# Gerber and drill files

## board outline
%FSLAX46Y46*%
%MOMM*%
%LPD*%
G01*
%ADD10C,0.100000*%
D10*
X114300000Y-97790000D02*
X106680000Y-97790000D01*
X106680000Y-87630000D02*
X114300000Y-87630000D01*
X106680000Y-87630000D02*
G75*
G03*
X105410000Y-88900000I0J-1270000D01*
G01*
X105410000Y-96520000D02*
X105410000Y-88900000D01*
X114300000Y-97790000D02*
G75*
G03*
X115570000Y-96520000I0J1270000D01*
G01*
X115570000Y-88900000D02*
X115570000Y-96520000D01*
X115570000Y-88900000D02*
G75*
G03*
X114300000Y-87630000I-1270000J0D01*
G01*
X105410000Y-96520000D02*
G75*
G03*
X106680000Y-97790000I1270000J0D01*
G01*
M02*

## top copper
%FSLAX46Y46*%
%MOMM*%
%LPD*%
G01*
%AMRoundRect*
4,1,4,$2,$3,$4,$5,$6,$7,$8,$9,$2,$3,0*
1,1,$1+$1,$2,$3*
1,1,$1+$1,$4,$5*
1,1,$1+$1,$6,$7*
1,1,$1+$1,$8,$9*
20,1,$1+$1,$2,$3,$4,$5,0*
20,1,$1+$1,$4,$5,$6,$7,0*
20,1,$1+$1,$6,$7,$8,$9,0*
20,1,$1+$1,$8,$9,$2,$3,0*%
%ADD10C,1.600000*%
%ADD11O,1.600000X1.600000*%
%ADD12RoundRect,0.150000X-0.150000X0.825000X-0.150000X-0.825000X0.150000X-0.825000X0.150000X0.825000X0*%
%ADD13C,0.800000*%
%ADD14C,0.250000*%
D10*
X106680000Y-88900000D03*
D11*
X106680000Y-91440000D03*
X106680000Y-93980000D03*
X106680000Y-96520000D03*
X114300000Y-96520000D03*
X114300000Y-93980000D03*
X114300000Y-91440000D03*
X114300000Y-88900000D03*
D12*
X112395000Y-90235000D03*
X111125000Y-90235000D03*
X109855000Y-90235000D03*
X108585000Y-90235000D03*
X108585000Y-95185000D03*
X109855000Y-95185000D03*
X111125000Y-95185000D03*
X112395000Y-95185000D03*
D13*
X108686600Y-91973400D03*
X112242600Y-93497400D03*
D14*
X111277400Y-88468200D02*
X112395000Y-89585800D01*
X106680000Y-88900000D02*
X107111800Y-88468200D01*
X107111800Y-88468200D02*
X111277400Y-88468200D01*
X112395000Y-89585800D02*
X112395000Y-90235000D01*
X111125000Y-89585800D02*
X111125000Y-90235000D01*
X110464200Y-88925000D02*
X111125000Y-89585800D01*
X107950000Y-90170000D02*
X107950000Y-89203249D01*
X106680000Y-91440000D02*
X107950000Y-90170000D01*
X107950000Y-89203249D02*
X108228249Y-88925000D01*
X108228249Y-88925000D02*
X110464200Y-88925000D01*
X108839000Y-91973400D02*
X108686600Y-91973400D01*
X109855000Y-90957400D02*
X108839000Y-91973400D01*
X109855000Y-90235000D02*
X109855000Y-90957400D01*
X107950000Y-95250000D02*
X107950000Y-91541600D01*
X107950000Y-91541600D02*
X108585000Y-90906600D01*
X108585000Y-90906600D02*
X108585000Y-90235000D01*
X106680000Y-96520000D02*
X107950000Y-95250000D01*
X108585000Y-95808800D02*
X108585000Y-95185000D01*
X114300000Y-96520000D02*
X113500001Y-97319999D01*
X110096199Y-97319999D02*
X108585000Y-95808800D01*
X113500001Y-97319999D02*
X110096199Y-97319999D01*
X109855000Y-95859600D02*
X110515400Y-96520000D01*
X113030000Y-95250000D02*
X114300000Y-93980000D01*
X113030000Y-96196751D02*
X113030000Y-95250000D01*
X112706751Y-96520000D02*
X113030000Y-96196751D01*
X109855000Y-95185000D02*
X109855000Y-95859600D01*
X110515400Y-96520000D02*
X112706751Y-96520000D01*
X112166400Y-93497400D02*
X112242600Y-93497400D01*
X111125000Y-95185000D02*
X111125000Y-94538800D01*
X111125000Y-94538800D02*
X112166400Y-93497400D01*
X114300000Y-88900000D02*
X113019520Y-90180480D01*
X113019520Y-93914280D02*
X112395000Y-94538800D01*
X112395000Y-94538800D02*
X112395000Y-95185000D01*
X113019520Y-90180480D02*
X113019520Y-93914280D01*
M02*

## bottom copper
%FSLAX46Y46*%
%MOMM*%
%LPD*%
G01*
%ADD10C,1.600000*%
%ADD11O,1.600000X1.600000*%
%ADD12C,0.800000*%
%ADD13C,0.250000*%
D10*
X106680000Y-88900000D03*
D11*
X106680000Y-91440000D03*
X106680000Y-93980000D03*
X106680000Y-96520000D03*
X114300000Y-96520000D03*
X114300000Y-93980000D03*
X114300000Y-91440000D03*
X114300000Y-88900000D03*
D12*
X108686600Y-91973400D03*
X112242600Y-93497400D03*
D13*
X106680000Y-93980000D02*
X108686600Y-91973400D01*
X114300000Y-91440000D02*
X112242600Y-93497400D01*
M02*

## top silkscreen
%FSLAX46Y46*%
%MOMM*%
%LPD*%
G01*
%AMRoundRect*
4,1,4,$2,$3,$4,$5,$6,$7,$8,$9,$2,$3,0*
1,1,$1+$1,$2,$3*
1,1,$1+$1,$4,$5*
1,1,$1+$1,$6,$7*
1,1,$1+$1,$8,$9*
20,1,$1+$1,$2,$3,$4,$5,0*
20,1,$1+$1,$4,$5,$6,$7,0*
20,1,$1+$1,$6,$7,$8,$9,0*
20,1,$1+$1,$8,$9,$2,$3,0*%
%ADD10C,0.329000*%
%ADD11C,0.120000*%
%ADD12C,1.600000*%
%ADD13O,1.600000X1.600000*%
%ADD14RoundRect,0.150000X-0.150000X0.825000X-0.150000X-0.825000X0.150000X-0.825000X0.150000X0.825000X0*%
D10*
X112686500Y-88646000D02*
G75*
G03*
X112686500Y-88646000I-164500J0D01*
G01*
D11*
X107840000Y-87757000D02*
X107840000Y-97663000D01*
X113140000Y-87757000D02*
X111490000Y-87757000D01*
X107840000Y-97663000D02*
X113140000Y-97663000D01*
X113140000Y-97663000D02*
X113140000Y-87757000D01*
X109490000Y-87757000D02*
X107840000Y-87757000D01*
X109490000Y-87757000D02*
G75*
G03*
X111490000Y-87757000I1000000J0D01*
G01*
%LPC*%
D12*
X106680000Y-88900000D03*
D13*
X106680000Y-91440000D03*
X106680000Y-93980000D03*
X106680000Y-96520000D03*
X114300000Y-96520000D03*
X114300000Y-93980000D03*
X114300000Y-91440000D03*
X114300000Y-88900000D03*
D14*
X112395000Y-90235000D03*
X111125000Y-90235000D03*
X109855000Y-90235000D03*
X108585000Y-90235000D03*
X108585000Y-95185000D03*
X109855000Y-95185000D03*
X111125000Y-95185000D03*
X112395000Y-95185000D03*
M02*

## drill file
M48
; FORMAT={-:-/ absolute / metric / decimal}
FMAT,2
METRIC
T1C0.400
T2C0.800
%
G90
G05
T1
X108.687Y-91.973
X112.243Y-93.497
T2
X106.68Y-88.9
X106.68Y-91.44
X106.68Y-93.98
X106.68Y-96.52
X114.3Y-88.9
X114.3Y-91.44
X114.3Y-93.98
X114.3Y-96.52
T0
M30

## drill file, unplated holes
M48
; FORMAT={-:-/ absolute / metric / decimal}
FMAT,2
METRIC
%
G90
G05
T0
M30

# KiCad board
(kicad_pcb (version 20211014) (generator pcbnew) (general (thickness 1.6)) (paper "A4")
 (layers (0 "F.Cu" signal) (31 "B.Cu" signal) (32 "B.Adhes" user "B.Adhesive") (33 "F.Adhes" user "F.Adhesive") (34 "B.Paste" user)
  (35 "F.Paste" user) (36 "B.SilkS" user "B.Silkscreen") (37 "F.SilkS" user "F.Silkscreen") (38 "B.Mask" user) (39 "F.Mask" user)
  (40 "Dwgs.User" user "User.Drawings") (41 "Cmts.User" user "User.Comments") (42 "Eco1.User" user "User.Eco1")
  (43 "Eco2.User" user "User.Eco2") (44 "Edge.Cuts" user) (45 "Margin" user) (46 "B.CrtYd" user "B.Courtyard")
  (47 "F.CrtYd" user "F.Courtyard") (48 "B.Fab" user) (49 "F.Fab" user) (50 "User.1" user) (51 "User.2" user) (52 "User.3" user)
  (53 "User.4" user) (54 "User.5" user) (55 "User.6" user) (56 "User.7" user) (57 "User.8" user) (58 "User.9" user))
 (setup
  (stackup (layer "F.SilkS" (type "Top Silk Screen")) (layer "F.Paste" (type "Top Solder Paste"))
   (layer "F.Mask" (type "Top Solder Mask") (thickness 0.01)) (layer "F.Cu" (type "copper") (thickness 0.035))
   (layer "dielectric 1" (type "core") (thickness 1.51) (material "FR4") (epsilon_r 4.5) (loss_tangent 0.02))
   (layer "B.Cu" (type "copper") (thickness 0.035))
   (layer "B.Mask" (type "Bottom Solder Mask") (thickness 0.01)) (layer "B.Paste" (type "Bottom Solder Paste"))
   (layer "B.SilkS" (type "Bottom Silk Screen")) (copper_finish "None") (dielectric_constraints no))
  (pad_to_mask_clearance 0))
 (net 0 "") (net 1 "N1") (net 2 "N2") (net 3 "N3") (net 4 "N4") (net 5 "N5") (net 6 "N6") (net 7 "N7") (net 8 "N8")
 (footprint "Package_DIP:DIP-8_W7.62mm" (layer "F.Cu") (at 106.68 88.9)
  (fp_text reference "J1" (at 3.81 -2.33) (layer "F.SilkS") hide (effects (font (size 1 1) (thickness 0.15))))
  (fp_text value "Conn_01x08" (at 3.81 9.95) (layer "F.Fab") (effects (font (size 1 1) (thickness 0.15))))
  (fp_line (start 1.16 -1.143) (end 1.16 8.763) (layer "F.SilkS") (width 0.12))
  (fp_line (start 6.46 -1.143) (end 4.81 -1.143) (layer "F.SilkS") (width 0.12))
  (fp_line (start 1.16 8.763) (end 6.46 8.763) (layer "F.SilkS") (width 0.12))
  (fp_line (start 6.46 8.763) (end 6.46 -1.143) (layer "F.SilkS") (width 0.12))
  (fp_line (start 2.81 -1.143) (end 1.16 -1.143) (layer "F.SilkS") (width 0.12))
  (fp_arc (start 4.81 -1.143) (mid 3.81 -0.143) (end 2.81 -1.143) (layer "F.SilkS") (width 0.12))
  (pad "1" thru_hole circle (at 0 0) (size 1.6 1.6) (drill 0.8) (layers *.Cu *.Mask) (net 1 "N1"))
  (pad "2" thru_hole oval (at 0 2.54) (size 1.6 1.6) (drill 0.8) (layers *.Cu *.Mask) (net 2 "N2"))
  (pad "3" thru_hole oval (at 0 5.08) (size 1.6 1.6) (drill 0.8) (layers *.Cu *.Mask) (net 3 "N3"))
  (pad "4" thru_hole oval (at 0 7.62) (size 1.6 1.6) (drill 0.8) (layers *.Cu *.Mask) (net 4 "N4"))
  (pad "5" thru_hole oval (at 7.62 7.62) (size 1.6 1.6) (drill 0.8) (layers *.Cu *.Mask) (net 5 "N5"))
  (pad "6" thru_hole oval (at 7.62 5.08) (size 1.6 1.6) (drill 0.8) (layers *.Cu *.Mask) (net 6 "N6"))
  (pad "7" thru_hole oval (at 7.62 2.54) (size 1.6 1.6) (drill 0.8) (layers *.Cu *.Mask) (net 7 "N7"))
  (pad "8" thru_hole oval (at 7.62 0) (size 1.6 1.6) (drill 0.8) (layers *.Cu *.Mask) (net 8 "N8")))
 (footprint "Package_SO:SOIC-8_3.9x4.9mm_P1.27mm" (layer "F.Cu") (at 110.49 92.71 -90)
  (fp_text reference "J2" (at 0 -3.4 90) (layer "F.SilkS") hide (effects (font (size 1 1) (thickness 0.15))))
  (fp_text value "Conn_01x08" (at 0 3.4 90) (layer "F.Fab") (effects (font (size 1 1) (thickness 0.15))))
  (pad "1" smd roundrect (at -2.475 -1.905 270) (size 1.95 0.6) (layers "F.Cu" "F.Paste" "F.Mask") (roundrect_rratio 0.25) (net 1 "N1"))
  (pad "2" smd roundrect (at -2.475 -0.635 270) (size 1.95 0.6) (layers "F.Cu" "F.Paste" "F.Mask") (roundrect_rratio 0.25) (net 2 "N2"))
  (pad "3" smd roundrect (at -2.475 0.635 270) (size 1.95 0.6) (layers "F.Cu" "F.Paste" "F.Mask") (roundrect_rratio 0.25) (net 3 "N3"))
  (pad "4" smd roundrect (at -2.475 1.905 270) (size 1.95 0.6) (layers "F.Cu" "F.Paste" "F.Mask") (roundrect_rratio 0.25) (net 4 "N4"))
  (pad "5" smd roundrect (at 2.475 1.905 270) (size 1.95 0.6) (layers "F.Cu" "F.Paste" "F.Mask") (roundrect_rratio 0.25) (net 5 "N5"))
  (pad "6" smd roundrect (at 2.475 0.635 270) (size 1.95 0.6) (layers "F.Cu" "F.Paste" "F.Mask") (roundrect_rratio 0.25) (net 6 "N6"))
  (pad "7" smd roundrect (at 2.475 -0.635 270) (size 1.95 0.6) (layers "F.Cu" "F.Paste" "F.Mask") (roundrect_rratio 0.25) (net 7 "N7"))
  (pad "8" smd roundrect (at 2.475 -1.905 270) (size 1.95 0.6) (layers "F.Cu" "F.Paste" "F.Mask") (roundrect_rratio 0.25) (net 8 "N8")))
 (gr_circle (center 112.522 88.646) (end 112.776 88.646) (layer "F.SilkS") (width 0.15) (fill solid))
 (gr_line (start 114.3 97.79) (end 106.68 97.79) (layer "Edge.Cuts") (width 0.1))
 (gr_line (start 106.68 87.63) (end 114.3 87.63) (layer "Edge.Cuts") (width 0.1))
 (gr_arc (start 105.41 88.9) (mid 105.781974 88.001974) (end 106.68 87.63) (layer "Edge.Cuts") (width 0.1))
 (gr_line (start 105.41 96.52) (end 105.41 88.9) (layer "Edge.Cuts") (width 0.1))
 (gr_arc (start 115.57 96.52) (mid 115.198026 97.418026) (end 114.3 97.79) (layer "Edge.Cuts") (width 0.1))
 (gr_line (start 115.57 88.9) (end 115.57 96.52) (layer "Edge.Cuts") (width 0.1))
 (gr_arc (start 114.3 87.63) (mid 115.198026 88.001974) (end 115.57 88.9) (layer "Edge.Cuts") (width 0.1))
 (gr_arc (start 106.68 97.79) (mid 105.781974 97.418026) (end 105.41 96.52) (layer "Edge.Cuts") (width 0.1))
 (segment (start 111.2774 88.4682) (end 112.395 89.5858) (width 0.25) (layer "F.Cu") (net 1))
 (segment (start 106.68 88.9) (end 107.1118 88.4682) (width 0.25) (layer "F.Cu") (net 1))
 (segment (start 107.1118 88.4682) (end 111.2774 88.4682) (width 0.25) (layer "F.Cu") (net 1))
 (segment (start 112.395 89.5858) (end 112.395 90.235) (width 0.25) (layer "F.Cu") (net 1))
 (segment (start 111.125 89.5858) (end 111.125 90.235) (width 0.25) (layer "F.Cu") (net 2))
 (segment (start 110.4642 88.925) (end 111.125 89.5858) (width 0.25) (layer "F.Cu") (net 2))
 (segment (start 107.95 90.17) (end 107.95 89.203249) (width 0.25) (layer "F.Cu") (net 2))
 (segment (start 106.68 91.44) (end 107.95 90.17) (width 0.25) (layer "F.Cu") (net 2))
 (segment (start 107.95 89.203249) (end 108.228249 88.925) (width 0.25) (layer "F.Cu") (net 2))
 (segment (start 108.228249 88.925) (end 110.4642 88.925) (width 0.25) (layer "F.Cu") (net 2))
 (segment (start 108.839 91.9734) (end 108.6866 91.9734) (width 0.25) (layer "F.Cu") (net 3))
 (segment (start 109.855 90.9574) (end 108.839 91.9734) (width 0.25) (layer "F.Cu") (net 3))
 (segment (start 109.855 90.235) (end 109.855 90.9574) (width 0.25) (layer "F.Cu") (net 3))
 (via (at 108.6866 91.9734) (size 0.8) (drill 0.4) (layers "F.Cu" "B.Cu") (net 3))
 (segment (start 106.68 93.98) (end 108.6866 91.9734) (width 0.25) (layer "B.Cu") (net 3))
 (segment (start 107.95 95.25) (end 107.95 91.5416) (width 0.25) (layer "F.Cu") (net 4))
 (segment (start 107.95 91.5416) (end 108.585 90.9066) (width 0.25) (layer "F.Cu") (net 4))
 (segment (start 108.585 90.9066) (end 108.585 90.235) (width 0.25) (layer "F.Cu") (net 4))
 (segment (start 106.68 96.52) (end 107.95 95.25) (width 0.25) (layer "F.Cu") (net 4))
 (segment (start 108.585 95.8088) (end 108.585 95.185) (width 0.25) (layer "F.Cu") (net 5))
 (segment (start 114.3 96.52) (end 113.500001 97.319999) (width 0.25) (layer "F.Cu") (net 5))
 (segment (start 110.096199 97.319999) (end 108.585 95.8088) (width 0.25) (layer "F.Cu") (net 5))
 (segment (start 113.500001 97.319999) (end 110.096199 97.319999) (width 0.25) (layer "F.Cu") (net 5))
 (segment (start 109.855 95.8596) (end 110.5154 96.52) (width 0.25) (layer "F.Cu") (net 6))
 (segment (start 113.03 95.25) (end 114.3 93.98) (width 0.25) (layer "F.Cu") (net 6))
 (segment (start 113.03 96.196751) (end 113.03 95.25) (width 0.25) (layer "F.Cu") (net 6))
 (segment (start 112.706751 96.52) (end 113.03 96.196751) (width 0.25) (layer "F.Cu") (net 6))
 (segment (start 109.855 95.185) (end 109.855 95.8596) (width 0.25) (layer "F.Cu") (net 6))
 (segment (start 110.5154 96.52) (end 112.706751 96.52) (width 0.25) (layer "F.Cu") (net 6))
 (segment (start 112.1664 93.4974) (end 112.2426 93.4974) (width 0.25) (layer "F.Cu") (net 7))
 (segment (start 111.125 95.185) (end 111.125 94.5388) (width 0.25) (layer "F.Cu") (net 7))
 (segment (start 111.125 94.5388) (end 112.1664 93.4974) (width 0.25) (layer "F.Cu") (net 7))
 (via (at 112.2426 93.4974) (size 0.8) (drill 0.4) (layers "F.Cu" "B.Cu") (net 7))
 (segment (start 114.3 91.44) (end 112.2426 93.4974) (width 0.25) (layer "B.Cu") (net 7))
 (segment (start 114.3 88.9) (end 113.01952 90.18048) (width 0.25) (layer "F.Cu") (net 8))
 (segment (start 113.01952 93.91428) (end 112.395 94.5388) (width 0.25) (layer "F.Cu") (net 8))
 (segment (start 112.395 94.5388) (end 112.395 95.185) (width 0.25) (layer "F.Cu") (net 8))
 (segment (start 113.01952 90.18048) (end 113.01952 93.91428) (width 0.25) (layer "F.Cu") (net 8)))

